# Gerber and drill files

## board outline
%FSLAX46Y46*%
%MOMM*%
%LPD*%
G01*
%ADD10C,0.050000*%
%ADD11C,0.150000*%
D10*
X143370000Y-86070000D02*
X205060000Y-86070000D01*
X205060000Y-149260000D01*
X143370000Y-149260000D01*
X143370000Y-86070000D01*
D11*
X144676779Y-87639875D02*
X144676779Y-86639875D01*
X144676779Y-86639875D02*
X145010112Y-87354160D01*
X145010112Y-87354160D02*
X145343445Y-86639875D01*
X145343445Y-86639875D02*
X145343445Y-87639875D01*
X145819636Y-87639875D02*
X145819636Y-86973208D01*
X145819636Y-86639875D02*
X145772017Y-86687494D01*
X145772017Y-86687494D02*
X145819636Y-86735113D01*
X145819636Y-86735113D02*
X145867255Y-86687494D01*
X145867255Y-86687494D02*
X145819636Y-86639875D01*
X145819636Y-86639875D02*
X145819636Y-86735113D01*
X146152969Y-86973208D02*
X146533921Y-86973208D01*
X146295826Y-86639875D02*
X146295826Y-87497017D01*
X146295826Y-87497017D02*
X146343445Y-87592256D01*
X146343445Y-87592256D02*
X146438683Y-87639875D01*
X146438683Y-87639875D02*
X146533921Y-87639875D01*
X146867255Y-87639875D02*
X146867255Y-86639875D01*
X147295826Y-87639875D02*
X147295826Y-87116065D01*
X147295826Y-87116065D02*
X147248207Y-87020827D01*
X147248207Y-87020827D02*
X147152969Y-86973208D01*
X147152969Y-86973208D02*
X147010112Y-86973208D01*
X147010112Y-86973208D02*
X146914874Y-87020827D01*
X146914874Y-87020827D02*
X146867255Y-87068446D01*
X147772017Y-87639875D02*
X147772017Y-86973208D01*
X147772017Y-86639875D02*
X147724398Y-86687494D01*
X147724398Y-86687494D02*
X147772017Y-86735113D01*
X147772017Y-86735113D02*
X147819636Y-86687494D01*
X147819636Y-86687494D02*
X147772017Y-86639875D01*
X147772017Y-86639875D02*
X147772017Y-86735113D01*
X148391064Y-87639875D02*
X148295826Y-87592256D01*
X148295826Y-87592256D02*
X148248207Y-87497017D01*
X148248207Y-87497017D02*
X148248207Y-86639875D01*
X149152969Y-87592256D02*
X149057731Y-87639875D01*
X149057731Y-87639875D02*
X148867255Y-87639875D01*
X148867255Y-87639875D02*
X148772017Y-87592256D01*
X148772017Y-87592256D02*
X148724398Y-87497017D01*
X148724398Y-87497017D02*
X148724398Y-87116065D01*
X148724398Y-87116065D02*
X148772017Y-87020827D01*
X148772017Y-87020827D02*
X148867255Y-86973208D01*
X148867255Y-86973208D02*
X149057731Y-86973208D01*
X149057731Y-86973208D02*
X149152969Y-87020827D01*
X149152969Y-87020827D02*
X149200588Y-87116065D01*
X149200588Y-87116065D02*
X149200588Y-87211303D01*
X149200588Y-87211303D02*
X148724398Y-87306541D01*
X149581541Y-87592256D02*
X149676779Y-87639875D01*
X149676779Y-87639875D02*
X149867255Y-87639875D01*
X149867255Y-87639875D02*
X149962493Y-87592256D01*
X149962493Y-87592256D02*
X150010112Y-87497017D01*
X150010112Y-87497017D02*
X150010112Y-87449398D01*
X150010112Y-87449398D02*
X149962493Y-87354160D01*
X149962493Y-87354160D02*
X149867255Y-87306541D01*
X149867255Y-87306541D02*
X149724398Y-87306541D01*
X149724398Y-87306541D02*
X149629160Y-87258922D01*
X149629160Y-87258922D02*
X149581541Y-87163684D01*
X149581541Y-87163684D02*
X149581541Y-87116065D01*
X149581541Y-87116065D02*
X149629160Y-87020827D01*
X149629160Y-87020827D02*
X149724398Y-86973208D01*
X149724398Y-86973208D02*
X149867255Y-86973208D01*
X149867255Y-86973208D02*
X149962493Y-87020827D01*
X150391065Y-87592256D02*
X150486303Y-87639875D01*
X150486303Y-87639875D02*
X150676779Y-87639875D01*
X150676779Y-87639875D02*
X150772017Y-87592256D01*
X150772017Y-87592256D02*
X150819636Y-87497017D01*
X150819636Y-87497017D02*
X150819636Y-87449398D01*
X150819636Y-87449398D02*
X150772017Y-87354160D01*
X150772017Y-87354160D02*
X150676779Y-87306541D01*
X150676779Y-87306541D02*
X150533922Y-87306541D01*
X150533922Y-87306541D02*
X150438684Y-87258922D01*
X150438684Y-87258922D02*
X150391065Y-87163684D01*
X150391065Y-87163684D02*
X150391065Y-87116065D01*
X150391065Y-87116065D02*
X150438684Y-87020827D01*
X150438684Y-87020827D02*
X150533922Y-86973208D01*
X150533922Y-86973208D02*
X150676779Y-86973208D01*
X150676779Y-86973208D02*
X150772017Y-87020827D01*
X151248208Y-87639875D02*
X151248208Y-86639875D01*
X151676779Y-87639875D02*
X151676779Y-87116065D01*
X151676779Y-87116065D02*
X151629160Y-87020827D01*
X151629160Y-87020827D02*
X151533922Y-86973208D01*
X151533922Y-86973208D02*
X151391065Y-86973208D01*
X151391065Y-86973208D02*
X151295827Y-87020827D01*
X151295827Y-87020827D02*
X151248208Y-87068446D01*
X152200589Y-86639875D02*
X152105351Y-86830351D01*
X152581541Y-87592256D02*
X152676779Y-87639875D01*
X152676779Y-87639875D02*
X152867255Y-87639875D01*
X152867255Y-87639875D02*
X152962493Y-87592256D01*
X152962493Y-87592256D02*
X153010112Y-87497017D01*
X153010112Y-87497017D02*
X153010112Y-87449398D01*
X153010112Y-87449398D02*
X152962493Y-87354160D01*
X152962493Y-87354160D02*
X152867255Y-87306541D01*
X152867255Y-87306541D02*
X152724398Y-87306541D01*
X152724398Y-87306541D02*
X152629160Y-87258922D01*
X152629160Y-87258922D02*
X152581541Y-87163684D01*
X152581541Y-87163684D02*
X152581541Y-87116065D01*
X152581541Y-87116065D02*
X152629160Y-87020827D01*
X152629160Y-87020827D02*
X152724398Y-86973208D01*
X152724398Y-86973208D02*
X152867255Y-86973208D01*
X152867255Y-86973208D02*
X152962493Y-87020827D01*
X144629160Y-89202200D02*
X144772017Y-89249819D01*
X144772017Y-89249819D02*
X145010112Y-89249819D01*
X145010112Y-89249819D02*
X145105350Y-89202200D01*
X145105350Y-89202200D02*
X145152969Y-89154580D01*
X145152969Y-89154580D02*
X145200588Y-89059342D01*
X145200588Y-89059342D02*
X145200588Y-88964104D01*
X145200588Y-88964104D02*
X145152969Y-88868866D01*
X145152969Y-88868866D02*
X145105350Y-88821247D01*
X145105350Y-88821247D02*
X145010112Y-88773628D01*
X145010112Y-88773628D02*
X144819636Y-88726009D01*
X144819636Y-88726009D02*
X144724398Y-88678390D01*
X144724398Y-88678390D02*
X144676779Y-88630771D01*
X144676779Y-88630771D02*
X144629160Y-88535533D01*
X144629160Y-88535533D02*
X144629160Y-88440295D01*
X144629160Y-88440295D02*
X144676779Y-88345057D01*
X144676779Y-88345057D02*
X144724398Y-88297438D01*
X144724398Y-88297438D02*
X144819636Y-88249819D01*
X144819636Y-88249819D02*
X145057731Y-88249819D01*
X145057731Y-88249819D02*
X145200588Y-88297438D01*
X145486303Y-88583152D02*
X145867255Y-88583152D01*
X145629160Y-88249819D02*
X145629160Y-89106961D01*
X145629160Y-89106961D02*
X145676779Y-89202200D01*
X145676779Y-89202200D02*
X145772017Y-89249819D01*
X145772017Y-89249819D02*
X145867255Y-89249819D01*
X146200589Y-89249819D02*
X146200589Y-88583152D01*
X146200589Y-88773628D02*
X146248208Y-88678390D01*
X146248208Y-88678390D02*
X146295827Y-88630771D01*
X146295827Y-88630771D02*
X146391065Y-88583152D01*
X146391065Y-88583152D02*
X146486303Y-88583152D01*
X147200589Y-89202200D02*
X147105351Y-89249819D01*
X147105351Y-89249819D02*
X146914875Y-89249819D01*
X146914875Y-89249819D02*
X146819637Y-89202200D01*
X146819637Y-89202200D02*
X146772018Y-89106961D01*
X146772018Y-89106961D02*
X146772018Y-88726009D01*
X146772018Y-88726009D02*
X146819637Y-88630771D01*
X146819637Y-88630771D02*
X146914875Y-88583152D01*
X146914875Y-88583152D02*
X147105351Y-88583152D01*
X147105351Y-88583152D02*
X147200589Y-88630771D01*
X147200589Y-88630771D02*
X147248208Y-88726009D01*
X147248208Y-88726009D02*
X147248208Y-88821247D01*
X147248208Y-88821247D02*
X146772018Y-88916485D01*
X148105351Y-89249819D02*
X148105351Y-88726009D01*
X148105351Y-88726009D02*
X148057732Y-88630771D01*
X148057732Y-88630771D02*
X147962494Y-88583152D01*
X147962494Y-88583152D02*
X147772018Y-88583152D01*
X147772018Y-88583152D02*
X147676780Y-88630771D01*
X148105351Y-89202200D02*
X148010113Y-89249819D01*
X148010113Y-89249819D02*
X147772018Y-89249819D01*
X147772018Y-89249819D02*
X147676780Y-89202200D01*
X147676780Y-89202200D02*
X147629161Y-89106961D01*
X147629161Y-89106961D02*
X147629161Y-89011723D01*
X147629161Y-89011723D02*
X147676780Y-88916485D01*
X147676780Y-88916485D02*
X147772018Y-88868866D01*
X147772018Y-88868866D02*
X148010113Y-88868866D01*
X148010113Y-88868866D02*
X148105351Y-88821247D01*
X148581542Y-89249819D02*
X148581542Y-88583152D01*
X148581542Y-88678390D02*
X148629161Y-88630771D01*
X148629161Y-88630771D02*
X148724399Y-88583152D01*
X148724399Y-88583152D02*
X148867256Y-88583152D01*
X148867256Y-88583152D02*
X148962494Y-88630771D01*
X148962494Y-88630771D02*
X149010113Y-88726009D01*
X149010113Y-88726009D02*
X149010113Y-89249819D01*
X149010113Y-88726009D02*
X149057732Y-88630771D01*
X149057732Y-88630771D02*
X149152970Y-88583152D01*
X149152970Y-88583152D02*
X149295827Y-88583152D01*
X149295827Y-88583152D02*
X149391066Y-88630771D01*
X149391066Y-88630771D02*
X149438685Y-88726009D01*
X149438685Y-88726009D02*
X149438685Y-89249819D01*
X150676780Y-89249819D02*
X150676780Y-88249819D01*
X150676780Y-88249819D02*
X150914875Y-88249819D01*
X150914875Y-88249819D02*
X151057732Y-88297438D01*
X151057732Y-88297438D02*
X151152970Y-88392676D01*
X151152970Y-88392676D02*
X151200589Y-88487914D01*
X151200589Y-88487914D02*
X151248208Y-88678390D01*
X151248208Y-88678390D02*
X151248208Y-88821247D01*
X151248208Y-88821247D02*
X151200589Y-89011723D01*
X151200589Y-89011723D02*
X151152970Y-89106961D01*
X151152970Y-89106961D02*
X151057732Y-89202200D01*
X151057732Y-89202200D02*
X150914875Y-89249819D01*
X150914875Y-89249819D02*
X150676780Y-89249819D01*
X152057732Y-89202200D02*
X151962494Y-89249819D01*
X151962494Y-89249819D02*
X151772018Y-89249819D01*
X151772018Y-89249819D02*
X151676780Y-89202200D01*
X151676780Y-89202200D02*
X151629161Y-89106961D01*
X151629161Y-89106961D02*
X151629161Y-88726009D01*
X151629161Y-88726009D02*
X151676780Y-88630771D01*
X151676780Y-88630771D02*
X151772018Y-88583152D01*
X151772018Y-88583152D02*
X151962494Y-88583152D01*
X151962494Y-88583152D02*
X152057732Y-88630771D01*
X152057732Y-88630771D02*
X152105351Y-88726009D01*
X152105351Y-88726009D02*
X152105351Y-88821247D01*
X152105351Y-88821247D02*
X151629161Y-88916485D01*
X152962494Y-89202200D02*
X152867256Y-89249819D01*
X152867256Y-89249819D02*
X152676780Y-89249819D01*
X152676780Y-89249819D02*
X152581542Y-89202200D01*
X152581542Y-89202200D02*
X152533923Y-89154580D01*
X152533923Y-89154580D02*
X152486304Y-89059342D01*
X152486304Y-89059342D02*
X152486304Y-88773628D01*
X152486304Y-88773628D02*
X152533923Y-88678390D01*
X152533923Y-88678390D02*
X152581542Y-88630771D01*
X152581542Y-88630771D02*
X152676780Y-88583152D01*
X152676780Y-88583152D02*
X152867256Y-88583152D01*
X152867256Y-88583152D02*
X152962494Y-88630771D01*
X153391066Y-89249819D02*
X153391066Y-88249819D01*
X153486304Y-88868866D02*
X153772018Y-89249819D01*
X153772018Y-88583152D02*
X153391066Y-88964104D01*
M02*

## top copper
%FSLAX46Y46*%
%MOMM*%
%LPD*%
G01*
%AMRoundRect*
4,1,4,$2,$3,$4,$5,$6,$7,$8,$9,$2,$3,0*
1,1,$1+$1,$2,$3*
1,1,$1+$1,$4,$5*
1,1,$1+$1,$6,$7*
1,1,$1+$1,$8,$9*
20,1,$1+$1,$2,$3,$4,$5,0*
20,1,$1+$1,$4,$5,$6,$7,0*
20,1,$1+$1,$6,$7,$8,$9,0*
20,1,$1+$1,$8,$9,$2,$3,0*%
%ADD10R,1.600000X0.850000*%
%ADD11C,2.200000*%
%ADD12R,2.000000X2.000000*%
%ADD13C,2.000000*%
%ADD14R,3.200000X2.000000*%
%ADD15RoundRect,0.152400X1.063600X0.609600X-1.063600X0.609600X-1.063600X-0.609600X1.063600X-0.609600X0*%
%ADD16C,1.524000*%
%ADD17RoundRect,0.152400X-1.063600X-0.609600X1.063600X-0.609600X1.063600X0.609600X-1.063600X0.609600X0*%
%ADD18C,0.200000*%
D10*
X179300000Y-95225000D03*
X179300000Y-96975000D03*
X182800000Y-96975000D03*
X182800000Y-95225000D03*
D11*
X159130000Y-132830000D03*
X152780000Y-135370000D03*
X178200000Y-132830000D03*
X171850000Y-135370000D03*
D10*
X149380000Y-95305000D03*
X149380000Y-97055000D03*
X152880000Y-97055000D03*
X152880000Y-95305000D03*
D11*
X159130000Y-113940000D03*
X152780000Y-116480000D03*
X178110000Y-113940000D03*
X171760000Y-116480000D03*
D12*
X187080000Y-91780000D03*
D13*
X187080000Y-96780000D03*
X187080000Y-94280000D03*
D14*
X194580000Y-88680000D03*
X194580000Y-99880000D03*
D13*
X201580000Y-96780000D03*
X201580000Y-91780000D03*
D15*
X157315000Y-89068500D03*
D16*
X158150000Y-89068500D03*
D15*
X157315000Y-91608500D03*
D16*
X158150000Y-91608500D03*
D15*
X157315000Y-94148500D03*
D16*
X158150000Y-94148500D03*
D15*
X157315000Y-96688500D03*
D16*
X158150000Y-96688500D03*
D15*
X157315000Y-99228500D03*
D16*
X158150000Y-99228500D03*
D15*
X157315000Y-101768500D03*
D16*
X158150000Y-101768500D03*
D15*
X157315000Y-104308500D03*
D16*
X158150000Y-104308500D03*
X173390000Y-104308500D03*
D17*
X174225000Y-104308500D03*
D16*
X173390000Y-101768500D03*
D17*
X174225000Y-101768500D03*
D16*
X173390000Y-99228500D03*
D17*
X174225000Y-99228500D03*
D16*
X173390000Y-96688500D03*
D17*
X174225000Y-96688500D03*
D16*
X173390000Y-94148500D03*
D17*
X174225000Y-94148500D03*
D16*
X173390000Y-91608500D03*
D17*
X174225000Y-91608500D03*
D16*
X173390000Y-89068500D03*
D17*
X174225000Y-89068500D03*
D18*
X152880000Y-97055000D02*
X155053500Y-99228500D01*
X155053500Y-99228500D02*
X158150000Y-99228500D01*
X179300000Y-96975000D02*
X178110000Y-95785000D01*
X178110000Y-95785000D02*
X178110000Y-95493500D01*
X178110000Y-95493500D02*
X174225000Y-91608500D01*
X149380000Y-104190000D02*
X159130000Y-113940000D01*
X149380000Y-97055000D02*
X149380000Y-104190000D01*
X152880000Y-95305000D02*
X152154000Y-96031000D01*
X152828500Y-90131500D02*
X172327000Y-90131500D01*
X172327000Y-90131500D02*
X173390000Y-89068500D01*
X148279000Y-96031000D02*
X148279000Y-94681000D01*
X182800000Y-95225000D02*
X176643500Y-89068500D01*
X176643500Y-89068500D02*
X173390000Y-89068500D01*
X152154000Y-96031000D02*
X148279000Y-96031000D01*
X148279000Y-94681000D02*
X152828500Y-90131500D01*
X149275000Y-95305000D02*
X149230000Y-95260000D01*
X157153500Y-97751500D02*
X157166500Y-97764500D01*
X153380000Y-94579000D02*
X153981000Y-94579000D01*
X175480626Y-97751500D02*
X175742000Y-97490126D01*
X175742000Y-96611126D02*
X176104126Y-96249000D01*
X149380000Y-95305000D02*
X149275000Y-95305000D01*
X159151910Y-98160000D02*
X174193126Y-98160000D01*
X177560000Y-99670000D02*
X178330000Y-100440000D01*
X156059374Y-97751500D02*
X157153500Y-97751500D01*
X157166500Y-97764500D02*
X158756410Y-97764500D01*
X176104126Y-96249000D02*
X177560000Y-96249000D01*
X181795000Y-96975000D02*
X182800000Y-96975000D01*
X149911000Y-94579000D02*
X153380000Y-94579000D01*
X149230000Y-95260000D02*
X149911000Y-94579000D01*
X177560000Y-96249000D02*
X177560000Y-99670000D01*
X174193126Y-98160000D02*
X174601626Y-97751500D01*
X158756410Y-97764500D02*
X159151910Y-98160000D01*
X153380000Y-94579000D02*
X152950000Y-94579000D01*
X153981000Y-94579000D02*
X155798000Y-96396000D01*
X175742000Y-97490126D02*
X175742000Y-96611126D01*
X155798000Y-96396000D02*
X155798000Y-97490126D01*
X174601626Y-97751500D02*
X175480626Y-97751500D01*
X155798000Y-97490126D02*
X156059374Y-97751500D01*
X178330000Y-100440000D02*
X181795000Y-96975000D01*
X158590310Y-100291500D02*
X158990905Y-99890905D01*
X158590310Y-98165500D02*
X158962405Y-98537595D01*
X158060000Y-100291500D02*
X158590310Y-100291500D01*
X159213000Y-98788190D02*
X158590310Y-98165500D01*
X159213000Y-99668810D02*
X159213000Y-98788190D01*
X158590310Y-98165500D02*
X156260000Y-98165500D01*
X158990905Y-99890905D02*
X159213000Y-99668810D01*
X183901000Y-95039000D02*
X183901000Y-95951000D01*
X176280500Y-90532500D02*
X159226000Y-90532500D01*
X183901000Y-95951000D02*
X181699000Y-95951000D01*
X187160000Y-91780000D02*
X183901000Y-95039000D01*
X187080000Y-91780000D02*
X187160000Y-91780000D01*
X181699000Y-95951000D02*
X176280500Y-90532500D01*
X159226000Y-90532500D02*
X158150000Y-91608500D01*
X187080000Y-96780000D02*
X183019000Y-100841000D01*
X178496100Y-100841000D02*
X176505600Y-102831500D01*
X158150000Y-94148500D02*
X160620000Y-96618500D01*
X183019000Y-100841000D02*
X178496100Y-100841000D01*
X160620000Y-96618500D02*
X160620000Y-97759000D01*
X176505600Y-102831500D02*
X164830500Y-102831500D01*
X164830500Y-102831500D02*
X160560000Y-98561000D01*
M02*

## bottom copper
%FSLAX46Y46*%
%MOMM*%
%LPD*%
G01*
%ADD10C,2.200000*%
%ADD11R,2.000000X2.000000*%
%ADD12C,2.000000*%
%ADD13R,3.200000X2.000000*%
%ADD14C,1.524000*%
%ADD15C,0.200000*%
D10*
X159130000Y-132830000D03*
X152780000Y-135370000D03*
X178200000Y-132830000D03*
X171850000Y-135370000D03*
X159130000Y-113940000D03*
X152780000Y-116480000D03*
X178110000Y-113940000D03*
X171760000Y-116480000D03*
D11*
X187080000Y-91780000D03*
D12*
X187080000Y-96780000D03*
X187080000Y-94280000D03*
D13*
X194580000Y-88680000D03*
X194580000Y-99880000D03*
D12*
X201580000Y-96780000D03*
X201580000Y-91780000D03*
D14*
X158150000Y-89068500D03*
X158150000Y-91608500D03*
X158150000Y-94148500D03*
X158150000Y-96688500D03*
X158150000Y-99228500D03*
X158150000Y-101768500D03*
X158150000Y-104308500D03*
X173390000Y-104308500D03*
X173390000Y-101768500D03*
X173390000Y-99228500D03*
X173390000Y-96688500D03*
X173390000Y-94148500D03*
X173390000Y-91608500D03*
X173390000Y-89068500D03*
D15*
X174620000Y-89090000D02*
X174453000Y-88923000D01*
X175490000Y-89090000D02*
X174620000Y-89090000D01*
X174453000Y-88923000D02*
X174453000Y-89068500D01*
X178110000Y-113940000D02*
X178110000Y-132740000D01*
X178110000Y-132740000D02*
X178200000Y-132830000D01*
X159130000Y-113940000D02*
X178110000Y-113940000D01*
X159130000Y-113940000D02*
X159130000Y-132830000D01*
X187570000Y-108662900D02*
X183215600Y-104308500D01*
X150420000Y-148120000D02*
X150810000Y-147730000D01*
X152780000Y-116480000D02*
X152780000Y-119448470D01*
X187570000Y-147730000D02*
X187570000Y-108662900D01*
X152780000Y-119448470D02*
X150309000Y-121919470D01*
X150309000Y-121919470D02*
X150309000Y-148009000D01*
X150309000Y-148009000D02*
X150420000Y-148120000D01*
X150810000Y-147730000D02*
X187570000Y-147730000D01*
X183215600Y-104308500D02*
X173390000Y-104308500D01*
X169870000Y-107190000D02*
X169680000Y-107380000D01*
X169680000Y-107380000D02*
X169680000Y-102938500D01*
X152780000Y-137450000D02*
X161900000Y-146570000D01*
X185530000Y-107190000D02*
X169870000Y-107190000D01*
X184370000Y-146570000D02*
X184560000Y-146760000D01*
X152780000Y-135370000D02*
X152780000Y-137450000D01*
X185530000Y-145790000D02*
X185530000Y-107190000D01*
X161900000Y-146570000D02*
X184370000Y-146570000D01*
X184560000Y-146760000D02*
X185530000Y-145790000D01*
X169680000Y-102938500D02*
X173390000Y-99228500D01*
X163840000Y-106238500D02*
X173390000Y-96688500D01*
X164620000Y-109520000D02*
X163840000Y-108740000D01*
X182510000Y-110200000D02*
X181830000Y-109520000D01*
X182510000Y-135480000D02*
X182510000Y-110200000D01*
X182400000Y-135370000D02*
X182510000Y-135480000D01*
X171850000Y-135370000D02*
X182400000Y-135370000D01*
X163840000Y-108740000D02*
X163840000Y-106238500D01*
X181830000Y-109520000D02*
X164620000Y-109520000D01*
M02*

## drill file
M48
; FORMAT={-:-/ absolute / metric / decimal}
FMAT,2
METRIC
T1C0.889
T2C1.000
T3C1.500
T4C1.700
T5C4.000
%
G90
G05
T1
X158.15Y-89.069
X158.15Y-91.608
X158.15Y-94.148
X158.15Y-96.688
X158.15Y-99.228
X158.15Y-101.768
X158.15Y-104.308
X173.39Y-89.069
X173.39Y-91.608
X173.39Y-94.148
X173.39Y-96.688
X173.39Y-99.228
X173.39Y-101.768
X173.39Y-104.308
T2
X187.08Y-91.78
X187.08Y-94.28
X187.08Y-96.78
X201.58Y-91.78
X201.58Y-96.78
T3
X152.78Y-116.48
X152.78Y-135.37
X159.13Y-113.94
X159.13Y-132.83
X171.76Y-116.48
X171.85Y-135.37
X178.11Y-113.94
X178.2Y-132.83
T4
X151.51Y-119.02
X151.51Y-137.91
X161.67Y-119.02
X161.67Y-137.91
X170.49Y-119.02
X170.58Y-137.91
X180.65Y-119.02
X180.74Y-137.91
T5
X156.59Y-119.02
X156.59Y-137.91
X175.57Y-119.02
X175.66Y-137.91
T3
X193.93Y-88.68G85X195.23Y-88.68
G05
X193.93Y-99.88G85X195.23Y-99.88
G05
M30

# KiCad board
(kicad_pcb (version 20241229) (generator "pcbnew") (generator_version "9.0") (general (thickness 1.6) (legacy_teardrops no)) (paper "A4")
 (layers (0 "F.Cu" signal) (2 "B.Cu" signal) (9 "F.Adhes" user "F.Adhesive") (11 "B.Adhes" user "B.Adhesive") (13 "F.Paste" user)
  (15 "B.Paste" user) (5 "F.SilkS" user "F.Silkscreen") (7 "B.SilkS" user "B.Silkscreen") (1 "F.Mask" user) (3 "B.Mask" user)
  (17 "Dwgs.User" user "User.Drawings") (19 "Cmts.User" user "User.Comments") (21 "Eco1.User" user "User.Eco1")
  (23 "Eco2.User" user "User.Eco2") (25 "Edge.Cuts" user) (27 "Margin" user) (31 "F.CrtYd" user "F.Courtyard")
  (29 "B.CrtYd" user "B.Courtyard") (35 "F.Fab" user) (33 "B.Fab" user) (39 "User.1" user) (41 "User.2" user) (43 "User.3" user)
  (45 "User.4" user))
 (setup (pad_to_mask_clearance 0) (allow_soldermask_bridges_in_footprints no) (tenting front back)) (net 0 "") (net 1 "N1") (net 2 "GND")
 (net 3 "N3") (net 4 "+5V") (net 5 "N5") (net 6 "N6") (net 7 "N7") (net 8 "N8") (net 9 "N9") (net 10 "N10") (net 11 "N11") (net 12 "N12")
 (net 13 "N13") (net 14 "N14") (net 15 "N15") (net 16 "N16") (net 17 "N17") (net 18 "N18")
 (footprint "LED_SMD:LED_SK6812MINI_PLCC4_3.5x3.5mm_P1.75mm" (layer "F.Cu") (at 181.05 96.1)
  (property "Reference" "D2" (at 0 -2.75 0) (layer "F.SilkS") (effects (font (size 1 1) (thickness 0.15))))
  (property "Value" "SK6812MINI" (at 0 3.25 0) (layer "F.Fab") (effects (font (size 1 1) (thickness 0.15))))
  (pad "1" smd rect (at -1.75 -0.875) (size 1.6 0.85) (layers "F.Cu" "F.Mask" "F.Paste") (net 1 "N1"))
  (pad "2" smd rect (at -1.75 0.875) (size 1.6 0.85) (layers "F.Cu" "F.Mask" "F.Paste") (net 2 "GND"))
  (pad "3" smd rect (at 1.75 0.875) (size 1.6 0.85) (layers "F.Cu" "F.Mask" "F.Paste") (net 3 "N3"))
  (pad "4" smd rect (at 1.75 -0.875) (size 1.6 0.85) (layers "F.Cu" "F.Mask" "F.Paste") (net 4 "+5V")))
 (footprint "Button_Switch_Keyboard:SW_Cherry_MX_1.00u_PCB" (layer "F.Cu") (at 159.13 132.83)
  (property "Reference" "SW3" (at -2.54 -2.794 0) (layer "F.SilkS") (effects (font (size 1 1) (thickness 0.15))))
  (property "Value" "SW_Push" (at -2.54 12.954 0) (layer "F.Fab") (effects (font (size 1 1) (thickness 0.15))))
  (pad "" np_thru_hole circle (at -7.62 5.08) (size 1.7 1.7) (drill 1.7) (layers "*.Cu" "*.Mask"))
  (pad "" np_thru_hole circle (at -2.54 5.08) (size 4 4) (drill 4) (layers "*.Cu" "*.Mask"))
  (pad "" np_thru_hole circle (at 2.54 5.08) (size 1.7 1.7) (drill 1.7) (layers "*.Cu" "*.Mask"))
  (pad "1" thru_hole circle (at 0 0) (size 2.2 2.2) (drill 1.5) (layers "*.Cu" "*.Mask") (remove_unused_layers no) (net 2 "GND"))
  (pad "2" thru_hole circle (at -6.35 2.54) (size 2.2 2.2) (drill 1.5) (layers "*.Cu" "*.Mask") (remove_unused_layers no) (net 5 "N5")))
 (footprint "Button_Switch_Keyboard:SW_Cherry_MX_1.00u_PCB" (layer "F.Cu") (at 178.2 132.83)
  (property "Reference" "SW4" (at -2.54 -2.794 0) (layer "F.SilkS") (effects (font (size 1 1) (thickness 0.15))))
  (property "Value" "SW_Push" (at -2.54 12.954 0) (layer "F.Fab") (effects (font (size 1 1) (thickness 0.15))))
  (pad "" np_thru_hole circle (at -7.62 5.08) (size 1.7 1.7) (drill 1.7) (layers "*.Cu" "*.Mask"))
  (pad "" np_thru_hole circle (at -2.54 5.08) (size 4 4) (drill 4) (layers "*.Cu" "*.Mask"))
  (pad "" np_thru_hole circle (at 2.54 5.08) (size 1.7 1.7) (drill 1.7) (layers "*.Cu" "*.Mask"))
  (pad "1" thru_hole circle (at 0 0) (size 2.2 2.2) (drill 1.5) (layers "*.Cu" "*.Mask") (remove_unused_layers no) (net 2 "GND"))
  (pad "2" thru_hole circle (at -6.35 2.54) (size 2.2 2.2) (drill 1.5) (layers "*.Cu" "*.Mask") (remove_unused_layers no) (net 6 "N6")))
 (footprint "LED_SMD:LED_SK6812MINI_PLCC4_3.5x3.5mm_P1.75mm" (layer "F.Cu") (at 151.13 96.18)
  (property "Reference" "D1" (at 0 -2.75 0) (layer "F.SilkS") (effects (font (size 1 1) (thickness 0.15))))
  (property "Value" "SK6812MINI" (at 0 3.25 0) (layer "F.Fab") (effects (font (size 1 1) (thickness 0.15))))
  (pad "1" smd rect (at -1.75 -0.875) (size 1.6 0.85) (layers "F.Cu" "F.Mask" "F.Paste") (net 3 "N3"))
  (pad "2" smd rect (at -1.75 0.875) (size 1.6 0.85) (layers "F.Cu" "F.Mask" "F.Paste") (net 2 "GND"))
  (pad "3" smd rect (at 1.75 0.875) (size 1.6 0.85) (layers "F.Cu" "F.Mask" "F.Paste") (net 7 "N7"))
  (pad "4" smd rect (at 1.75 -0.875) (size 1.6 0.85) (layers "F.Cu" "F.Mask" "F.Paste") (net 4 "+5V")))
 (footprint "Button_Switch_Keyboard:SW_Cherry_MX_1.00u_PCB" (layer "F.Cu") (at 159.13 113.94)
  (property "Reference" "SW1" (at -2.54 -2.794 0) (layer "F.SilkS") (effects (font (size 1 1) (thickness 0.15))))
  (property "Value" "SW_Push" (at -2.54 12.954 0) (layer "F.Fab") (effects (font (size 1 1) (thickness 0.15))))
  (pad "" np_thru_hole circle (at -7.62 5.08) (size 1.7 1.7) (drill 1.7) (layers "*.Cu" "*.Mask"))
  (pad "" np_thru_hole circle (at -2.54 5.08) (size 4 4) (drill 4) (layers "*.Cu" "*.Mask"))
  (pad "" np_thru_hole circle (at 2.54 5.08) (size 1.7 1.7) (drill 1.7) (layers "*.Cu" "*.Mask"))
  (pad "1" thru_hole circle (at 0 0) (size 2.2 2.2) (drill 1.5) (layers "*.Cu" "*.Mask") (remove_unused_layers no) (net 2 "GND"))
  (pad "2" thru_hole circle (at -6.35 2.54) (size 2.2 2.2) (drill 1.5) (layers "*.Cu" "*.Mask") (remove_unused_layers no) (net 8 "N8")))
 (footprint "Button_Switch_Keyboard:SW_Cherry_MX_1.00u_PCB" (layer "F.Cu") (at 178.11 113.94)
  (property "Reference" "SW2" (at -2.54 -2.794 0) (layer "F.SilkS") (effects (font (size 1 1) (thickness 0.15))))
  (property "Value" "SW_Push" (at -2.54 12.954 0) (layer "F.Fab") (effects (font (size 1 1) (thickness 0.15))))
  (pad "" np_thru_hole circle (at -7.62 5.08) (size 1.7 1.7) (drill 1.7) (layers "*.Cu" "*.Mask"))
  (pad "" np_thru_hole circle (at -2.54 5.08) (size 4 4) (drill 4) (layers "*.Cu" "*.Mask"))
  (pad "" np_thru_hole circle (at 2.54 5.08) (size 1.7 1.7) (drill 1.7) (layers "*.Cu" "*.Mask"))
  (pad "1" thru_hole circle (at 0 0) (size 2.2 2.2) (drill 1.5) (layers "*.Cu" "*.Mask") (remove_unused_layers no) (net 2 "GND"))
  (pad "2" thru_hole circle (at -6.35 2.54) (size 2.2 2.2) (drill 1.5) (layers "*.Cu" "*.Mask") (remove_unused_layers no) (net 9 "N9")))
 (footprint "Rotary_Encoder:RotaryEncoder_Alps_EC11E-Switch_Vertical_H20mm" (layer "F.Cu") (at 187.08 91.78)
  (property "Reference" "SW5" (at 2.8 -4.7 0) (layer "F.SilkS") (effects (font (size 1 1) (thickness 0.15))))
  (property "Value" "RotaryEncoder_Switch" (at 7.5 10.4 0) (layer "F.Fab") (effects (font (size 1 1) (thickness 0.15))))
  (pad "A" thru_hole rect (at 0 0) (size 2 2) (drill 1) (layers "*.Cu" "*.Mask") (remove_unused_layers no) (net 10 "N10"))
  (pad "B" thru_hole circle (at 0 5) (size 2 2) (drill 1) (layers "*.Cu" "*.Mask") (remove_unused_layers no) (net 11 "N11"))
  (pad "C" thru_hole circle (at 0 2.5) (size 2 2) (drill 1) (layers "*.Cu" "*.Mask") (remove_unused_layers no) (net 2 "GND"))
  (pad "MP" thru_hole rect (at 7.5 -3.1) (size 3.2 2) (drill oval 2.8 1.5) (layers "*.Cu" "*.Mask") (remove_unused_layers no))
  (pad "MP" thru_hole rect (at 7.5 8.1) (size 3.2 2) (drill oval 2.8 1.5) (layers "*.Cu" "*.Mask") (remove_unused_layers no))
  (pad "S1" thru_hole circle (at 14.5 5) (size 2 2) (drill 1) (layers "*.Cu" "*.Mask") (remove_unused_layers no) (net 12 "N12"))
  (pad "S2" thru_hole circle (at 14.5 0) (size 2 2) (drill 1) (layers "*.Cu" "*.Mask") (remove_unused_layers no) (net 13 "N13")))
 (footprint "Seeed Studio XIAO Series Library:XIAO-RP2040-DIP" (layer "F.Cu") (at 165.77 96.6885)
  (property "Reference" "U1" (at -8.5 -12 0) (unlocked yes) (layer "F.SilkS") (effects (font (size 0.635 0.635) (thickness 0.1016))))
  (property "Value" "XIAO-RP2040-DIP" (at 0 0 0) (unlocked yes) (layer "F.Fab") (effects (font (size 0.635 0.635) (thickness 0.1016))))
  (pad "1" smd roundrect (at -8.455 -7.62 180) (size 2.432 1.524) (layers "F.Cu" "F.Mask") (roundrect_rratio 0.1) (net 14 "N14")
   (thermal_bridge_angle 45))
  (pad "1" thru_hole circle (at -7.62 -7.62 180) (size 1.524 1.524) (drill 0.889) (layers "*.Cu" "*.Mask") (remove_unused_layers no)
   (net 14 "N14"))
  (pad "2" smd roundrect (at -8.455 -5.08 180) (size 2.432 1.524) (layers "F.Cu" "F.Mask") (roundrect_rratio 0.1) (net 10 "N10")
   (thermal_bridge_angle 45))
  (pad "2" thru_hole circle (at -7.62 -5.08 180) (size 1.524 1.524) (drill 0.889) (layers "*.Cu" "*.Mask") (remove_unused_layers no)
   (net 10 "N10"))
  (pad "3" smd roundrect (at -8.455 -2.54 180) (size 2.432 1.524) (layers "F.Cu" "F.Mask") (roundrect_rratio 0.1) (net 11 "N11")
   (thermal_bridge_angle 45))
  (pad "3" thru_hole circle (at -7.62 -2.54 180) (size 1.524 1.524) (drill 0.889) (layers "*.Cu" "*.Mask") (remove_unused_layers no)
   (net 11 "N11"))
  (pad "4" smd roundrect (at -8.455 0 180) (size 2.432 1.524) (layers "F.Cu" "F.Mask") (roundrect_rratio 0.1) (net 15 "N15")
   (thermal_bridge_angle 45))
  (pad "4" thru_hole circle (at -7.62 0 180) (size 1.524 1.524) (drill 0.889) (layers "*.Cu" "*.Mask") (remove_unused_layers no)
   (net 15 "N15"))
  (pad "5" smd roundrect (at -8.455 2.54 180) (size 2.432 1.524) (layers "F.Cu" "F.Mask") (roundrect_rratio 0.1) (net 7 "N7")
   (thermal_bridge_angle 45))
  (pad "5" thru_hole circle (at -7.62 2.54 180) (size 1.524 1.524) (drill 0.889) (layers "*.Cu" "*.Mask") (remove_unused_layers no)
   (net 7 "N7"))
  (pad "6" smd roundrect (at -8.455 5.08 180) (size 2.432 1.524) (layers "F.Cu" "F.Mask") (roundrect_rratio 0.1) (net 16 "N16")
   (thermal_bridge_angle 45))
  (pad "6" thru_hole circle (at -7.62 5.08 180) (size 1.524 1.524) (drill 0.889) (layers "*.Cu" "*.Mask") (remove_unused_layers no)
   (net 16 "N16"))
  (pad "7" smd roundrect (at -8.455 7.62 180) (size 2.432 1.524) (layers "F.Cu" "F.Mask") (roundrect_rratio 0.1) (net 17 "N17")
   (thermal_bridge_angle 45))
  (pad "7" thru_hole circle (at -7.62 7.62 180) (size 1.524 1.524) (drill 0.889) (layers "*.Cu" "*.Mask") (remove_unused_layers no)
   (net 17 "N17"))
  (pad "8" thru_hole circle (at 7.62 7.62) (size 1.524 1.524) (drill 0.889) (layers "*.Cu" "*.Mask") (remove_unused_layers no) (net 8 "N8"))
  (pad "8" smd roundrect (at 8.455 7.62) (size 2.432 1.524) (layers "F.Cu" "F.Mask") (roundrect_rratio 0.1) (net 8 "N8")
   (thermal_bridge_angle 45))
  (pad "9" thru_hole circle (at 7.62 5.08) (size 1.524 1.524) (drill 0.889) (layers "*.Cu" "*.Mask") (remove_unused_layers no) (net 9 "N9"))
  (pad "9" smd roundrect (at 8.455 5.08) (size 2.432 1.524) (layers "F.Cu" "F.Mask") (roundrect_rratio 0.1) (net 9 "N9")
   (thermal_bridge_angle 45))
  (pad "10" thru_hole circle (at 7.62 2.54) (size 1.524 1.524) (drill 0.889) (layers "*.Cu" "*.Mask") (remove_unused_layers no) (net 5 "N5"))
  (pad "10" smd roundrect (at 8.455 2.54) (size 2.432 1.524) (layers "F.Cu" "F.Mask") (roundrect_rratio 0.1) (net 5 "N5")
   (thermal_bridge_angle 45))
  (pad "11" thru_hole circle (at 7.62 0) (size 1.524 1.524) (drill 0.889) (layers "*.Cu" "*.Mask") (remove_unused_layers no) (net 6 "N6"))
  (pad "11" smd roundrect (at 8.455 0) (size 2.432 1.524) (layers "F.Cu" "F.Mask") (roundrect_rratio 0.1) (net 6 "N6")
   (thermal_bridge_angle 45))
  (pad "12" thru_hole circle (at 7.62 -2.54) (size 1.524 1.524) (drill 0.889) (layers "*.Cu" "*.Mask") (remove_unused_layers no)
   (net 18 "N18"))
  (pad "12" smd roundrect (at 8.455 -2.54) (size 2.432 1.524) (layers "F.Cu" "F.Mask") (roundrect_rratio 0.1) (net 18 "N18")
   (thermal_bridge_angle 45))
  (pad "13" thru_hole circle (at 7.62 -5.08) (size 1.524 1.524) (drill 0.889) (layers "*.Cu" "*.Mask") (remove_unused_layers no)
   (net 2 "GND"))
  (pad "13" smd roundrect (at 8.455 -5.08) (size 2.432 1.524) (layers "F.Cu" "F.Mask") (roundrect_rratio 0.1) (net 2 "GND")
   (thermal_bridge_angle 45))
  (pad "14" thru_hole circle (at 7.62 -7.62) (size 1.524 1.524) (drill 0.889) (layers "*.Cu" "*.Mask") (remove_unused_layers no)
   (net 4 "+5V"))
  (pad "14" smd roundrect (at 8.455 -7.62) (size 2.432 1.524) (layers "F.Cu" "F.Mask") (roundrect_rratio 0.1) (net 4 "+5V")
   (thermal_bridge_angle 45)))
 (gr_rect (start 143.37 86.07) (end 205.06 149.26) (stroke (width 0.05) (type default)) (fill no) (layer "Edge.Cuts"))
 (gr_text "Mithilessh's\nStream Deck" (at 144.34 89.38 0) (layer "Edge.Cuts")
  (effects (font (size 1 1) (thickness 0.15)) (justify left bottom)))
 (segment (start 174.62 89.09) (end 174.453 88.923) (width 0.2) (layer "B.Cu") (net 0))
 (segment (start 175.49 89.09) (end 174.62 89.09) (width 0.2) (layer "B.Cu") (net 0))
 (segment (start 174.453 88.923) (end 174.453 89.0685) (width 0.2) (layer "B.Cu") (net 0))
 (segment (start 152.88 97.055) (end 155.0535 99.2285) (width 0.2) (layer "F.Cu") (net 7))
 (segment (start 155.0535 99.2285) (end 158.15 99.2285) (width 0.2) (layer "F.Cu") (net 7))
 (segment (start 179.3 96.975) (end 178.11 95.785) (width 0.2) (layer "F.Cu") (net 2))
 (segment (start 178.11 95.785) (end 178.11 95.4935) (width 0.2) (layer "F.Cu") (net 2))
 (segment (start 178.11 95.4935) (end 174.225 91.6085) (width 0.2) (layer "F.Cu") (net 2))
 (segment (start 149.38 104.19) (end 159.13 113.94) (width 0.2) (layer "F.Cu") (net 2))
 (segment (start 149.38 97.055) (end 149.38 104.19) (width 0.2) (layer "F.Cu") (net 2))
 (segment (start 178.11 113.94) (end 178.11 132.74) (width 0.2) (layer "B.Cu") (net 2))
 (segment (start 178.11 132.74) (end 178.2 132.83) (width 0.2) (layer "B.Cu") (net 2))
 (segment (start 159.13 113.94) (end 178.11 113.94) (width 0.2) (layer "B.Cu") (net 2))
 (segment (start 159.13 113.94) (end 159.13 132.83) (width 0.2) (layer "B.Cu") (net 2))
 (segment (start 152.88 95.305) (end 152.154 96.031) (width 0.2) (layer "F.Cu") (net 4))
 (segment (start 152.8285 90.1315) (end 172.327 90.1315) (width 0.2) (layer "F.Cu") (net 4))
 (segment (start 172.327 90.1315) (end 173.39 89.0685) (width 0.2) (layer "F.Cu") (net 4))
 (segment (start 148.279 96.031) (end 148.279 94.681) (width 0.2) (layer "F.Cu") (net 4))
 (segment (start 182.8 95.225) (end 176.6435 89.0685) (width 0.2) (layer "F.Cu") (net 4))
 (segment (start 176.6435 89.0685) (end 173.39 89.0685) (width 0.2) (layer "F.Cu") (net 4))
 (segment (start 152.154 96.031) (end 148.279 96.031) (width 0.2) (layer "F.Cu") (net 4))
 (segment (start 148.279 94.681) (end 152.8285 90.1315) (width 0.2) (layer "F.Cu") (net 4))
 (segment (start 149.275 95.305) (end 149.23 95.26) (width 0.2) (layer "F.Cu") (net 3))
 (segment (start 157.1535 97.7515) (end 157.1665 97.7645) (width 0.2) (layer "F.Cu") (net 3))
 (segment (start 153.38 94.579) (end 153.981 94.579) (width 0.2) (layer "F.Cu") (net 3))
 (segment (start 175.480626 97.7515) (end 175.742 97.490126) (width 0.2) (layer "F.Cu") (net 3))
 (segment (start 175.742 96.611126) (end 176.104126 96.249) (width 0.2) (layer "F.Cu") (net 3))
 (segment (start 149.38 95.305) (end 149.275 95.305) (width 0.2) (layer "F.Cu") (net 3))
 (segment (start 159.15191 98.16) (end 174.193126 98.16) (width 0.2) (layer "F.Cu") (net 3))
 (segment (start 177.56 99.67) (end 178.33 100.44) (width 0.2) (layer "F.Cu") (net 3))
 (segment (start 156.059374 97.7515) (end 157.1535 97.7515) (width 0.2) (layer "F.Cu") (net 3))
 (segment (start 157.1665 97.7645) (end 158.75641 97.7645) (width 0.2) (layer "F.Cu") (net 3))
 (segment (start 176.104126 96.249) (end 177.56 96.249) (width 0.2) (layer "F.Cu") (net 3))
 (segment (start 181.795 96.975) (end 182.8 96.975) (width 0.2) (layer "F.Cu") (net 3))
 (segment (start 149.911 94.579) (end 153.38 94.579) (width 0.2) (layer "F.Cu") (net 3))
 (segment (start 149.23 95.26) (end 149.911 94.579) (width 0.2) (layer "F.Cu") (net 3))
 (segment (start 177.56 96.249) (end 177.56 99.67) (width 0.2) (layer "F.Cu") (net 3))
 (segment (start 174.193126 98.16) (end 174.601626 97.7515) (width 0.2) (layer "F.Cu") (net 3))
 (segment (start 158.75641 97.7645) (end 159.15191 98.16) (width 0.2) (layer "F.Cu") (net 3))
 (segment (start 153.38 94.579) (end 152.95 94.579) (width 0.2) (layer "F.Cu") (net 3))
 (segment (start 153.981 94.579) (end 155.798 96.396) (width 0.2) (layer "F.Cu") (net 3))
 (segment (start 175.742 97.490126) (end 175.742 96.611126) (width 0.2) (layer "F.Cu") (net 3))
 (segment (start 155.798 96.396) (end 155.798 97.490126) (width 0.2) (layer "F.Cu") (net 3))
 (segment (start 174.601626 97.7515) (end 175.480626 97.7515) (width 0.2) (layer "F.Cu") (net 3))
 (segment (start 155.798 97.490126) (end 156.059374 97.7515) (width 0.2) (layer "F.Cu") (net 3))
 (segment (start 178.33 100.44) (end 181.795 96.975) (width 0.2) (layer "F.Cu") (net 3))
 (segment (start 158.59031 100.2915) (end 158.990905 99.890905) (width 0.2) (layer "F.Cu") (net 1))
 (segment (start 158.59031 98.1655) (end 158.962405 98.537595) (width 0.2) (layer "F.Cu") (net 1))
 (segment (start 158.06 100.2915) (end 158.59031 100.2915) (width 0.2) (layer "F.Cu") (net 1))
 (segment (start 159.213 98.78819) (end 158.59031 98.1655) (width 0.2) (layer "F.Cu") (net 1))
 (segment (start 159.213 99.66881) (end 159.213 98.78819) (width 0.2) (layer "F.Cu") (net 1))
 (segment (start 158.59031 98.1655) (end 156.26 98.1655) (width 0.2) (layer "F.Cu") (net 1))
 (segment (start 158.990905 99.890905) (end 159.213 99.66881) (width 0.2) (layer "F.Cu") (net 1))
 (segment (start 187.57 108.6629) (end 183.2156 104.3085) (width 0.2) (layer "B.Cu") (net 8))
 (segment (start 150.42 148.12) (end 150.81 147.73) (width 0.2) (layer "B.Cu") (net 8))
 (segment (start 152.78 116.48) (end 152.78 119.44847) (width 0.2) (layer "B.Cu") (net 8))
 (segment (start 187.57 147.73) (end 187.57 108.6629) (width 0.2) (layer "B.Cu") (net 8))
 (segment (start 152.78 119.44847) (end 150.309 121.91947) (width 0.2) (layer "B.Cu") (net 8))
 (segment (start 150.309 121.91947) (end 150.309 148.009) (width 0.2) (layer "B.Cu") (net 8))
 (segment (start 150.309 148.009) (end 150.42 148.12) (width 0.2) (layer "B.Cu") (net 8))
 (segment (start 150.81 147.73) (end 187.57 147.73) (width 0.2) (layer "B.Cu") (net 8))
 (segment (start 183.2156 104.3085) (end 173.39 104.3085) (width 0.2) (layer "B.Cu") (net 8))
 (segment (start 169.87 107.19) (end 169.68 107.38) (width 0.2) (layer "B.Cu") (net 5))
 (segment (start 169.68 107.38) (end 169.68 102.9385) (width 0.2) (layer "B.Cu") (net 5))
 (segment (start 152.78 137.45) (end 161.9 146.57) (width 0.2) (layer "B.Cu") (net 5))
 (segment (start 185.53 107.19) (end 169.87 107.19) (width 0.2) (layer "B.Cu") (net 5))
 (segment (start 184.37 146.57) (end 184.56 146.76) (width 0.2) (layer "B.Cu") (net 5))
 (segment (start 152.78 135.37) (end 152.78 137.45) (width 0.2) (layer "B.Cu") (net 5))
 (segment (start 185.53 145.79) (end 185.53 107.19) (width 0.2) (layer "B.Cu") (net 5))
 (segment (start 161.9 146.57) (end 184.37 146.57) (width 0.2) (layer "B.Cu") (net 5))
 (segment (start 184.56 146.76) (end 185.53 145.79) (width 0.2) (layer "B.Cu") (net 5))
 (segment (start 169.68 102.9385) (end 173.39 99.2285) (width 0.2) (layer "B.Cu") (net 5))
 (segment (start 163.84 106.2385) (end 173.39 96.6885) (width 0.2) (layer "B.Cu") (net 6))
 (segment (start 164.62 109.52) (end 163.84 108.74) (width 0.2) (layer "B.Cu") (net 6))
 (segment (start 182.51 110.2) (end 181.83 109.52) (width 0.2) (layer "B.Cu") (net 6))
 (segment (start 182.51 135.48) (end 182.51 110.2) (width 0.2) (layer "B.Cu") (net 6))
 (segment (start 182.4 135.37) (end 182.51 135.48) (width 0.2) (layer "B.Cu") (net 6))
 (segment (start 171.85 135.37) (end 182.4 135.37) (width 0.2) (layer "B.Cu") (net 6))
 (segment (start 163.84 108.74) (end 163.84 106.2385) (width 0.2) (layer "B.Cu") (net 6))
 (segment (start 181.83 109.52) (end 164.62 109.52) (width 0.2) (layer "B.Cu") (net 6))
 (segment (start 183.901 95.039) (end 183.901 95.951) (width 0.2) (layer "F.Cu") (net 10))
 (segment (start 176.2805 90.5325) (end 159.226 90.5325) (width 0.2) (layer "F.Cu") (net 10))
 (segment (start 183.901 95.951) (end 181.699 95.951) (width 0.2) (layer "F.Cu") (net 10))
 (segment (start 187.16 91.78) (end 183.901 95.039) (width 0.2) (layer "F.Cu") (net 10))
 (segment (start 187.08 91.78) (end 187.16 91.78) (width 0.2) (layer "F.Cu") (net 10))
 (segment (start 181.699 95.951) (end 176.2805 90.5325) (width 0.2) (layer "F.Cu") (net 10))
 (segment (start 159.226 90.5325) (end 158.15 91.6085) (width 0.2) (layer "F.Cu") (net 10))
 (segment (start 187.08 96.78) (end 183.019 100.841) (width 0.2) (layer "F.Cu") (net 11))
 (segment (start 178.4961 100.841) (end 176.5056 102.8315) (width 0.2) (layer "F.Cu") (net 11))
 (segment (start 158.15 94.1485) (end 160.62 96.6185) (width 0.2) (layer "F.Cu") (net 11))
 (segment (start 183.019 100.841) (end 178.4961 100.841) (width 0.2) (layer "F.Cu") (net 11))
 (segment (start 160.62 96.6185) (end 160.62 97.759) (width 0.2) (layer "F.Cu") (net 11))
 (segment (start 176.5056 102.8315) (end 164.8305 102.8315) (width 0.2) (layer "F.Cu") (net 11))
 (segment (start 164.8305 102.8315) (end 160.56 98.561) (width 0.2) (layer "F.Cu") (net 11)))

